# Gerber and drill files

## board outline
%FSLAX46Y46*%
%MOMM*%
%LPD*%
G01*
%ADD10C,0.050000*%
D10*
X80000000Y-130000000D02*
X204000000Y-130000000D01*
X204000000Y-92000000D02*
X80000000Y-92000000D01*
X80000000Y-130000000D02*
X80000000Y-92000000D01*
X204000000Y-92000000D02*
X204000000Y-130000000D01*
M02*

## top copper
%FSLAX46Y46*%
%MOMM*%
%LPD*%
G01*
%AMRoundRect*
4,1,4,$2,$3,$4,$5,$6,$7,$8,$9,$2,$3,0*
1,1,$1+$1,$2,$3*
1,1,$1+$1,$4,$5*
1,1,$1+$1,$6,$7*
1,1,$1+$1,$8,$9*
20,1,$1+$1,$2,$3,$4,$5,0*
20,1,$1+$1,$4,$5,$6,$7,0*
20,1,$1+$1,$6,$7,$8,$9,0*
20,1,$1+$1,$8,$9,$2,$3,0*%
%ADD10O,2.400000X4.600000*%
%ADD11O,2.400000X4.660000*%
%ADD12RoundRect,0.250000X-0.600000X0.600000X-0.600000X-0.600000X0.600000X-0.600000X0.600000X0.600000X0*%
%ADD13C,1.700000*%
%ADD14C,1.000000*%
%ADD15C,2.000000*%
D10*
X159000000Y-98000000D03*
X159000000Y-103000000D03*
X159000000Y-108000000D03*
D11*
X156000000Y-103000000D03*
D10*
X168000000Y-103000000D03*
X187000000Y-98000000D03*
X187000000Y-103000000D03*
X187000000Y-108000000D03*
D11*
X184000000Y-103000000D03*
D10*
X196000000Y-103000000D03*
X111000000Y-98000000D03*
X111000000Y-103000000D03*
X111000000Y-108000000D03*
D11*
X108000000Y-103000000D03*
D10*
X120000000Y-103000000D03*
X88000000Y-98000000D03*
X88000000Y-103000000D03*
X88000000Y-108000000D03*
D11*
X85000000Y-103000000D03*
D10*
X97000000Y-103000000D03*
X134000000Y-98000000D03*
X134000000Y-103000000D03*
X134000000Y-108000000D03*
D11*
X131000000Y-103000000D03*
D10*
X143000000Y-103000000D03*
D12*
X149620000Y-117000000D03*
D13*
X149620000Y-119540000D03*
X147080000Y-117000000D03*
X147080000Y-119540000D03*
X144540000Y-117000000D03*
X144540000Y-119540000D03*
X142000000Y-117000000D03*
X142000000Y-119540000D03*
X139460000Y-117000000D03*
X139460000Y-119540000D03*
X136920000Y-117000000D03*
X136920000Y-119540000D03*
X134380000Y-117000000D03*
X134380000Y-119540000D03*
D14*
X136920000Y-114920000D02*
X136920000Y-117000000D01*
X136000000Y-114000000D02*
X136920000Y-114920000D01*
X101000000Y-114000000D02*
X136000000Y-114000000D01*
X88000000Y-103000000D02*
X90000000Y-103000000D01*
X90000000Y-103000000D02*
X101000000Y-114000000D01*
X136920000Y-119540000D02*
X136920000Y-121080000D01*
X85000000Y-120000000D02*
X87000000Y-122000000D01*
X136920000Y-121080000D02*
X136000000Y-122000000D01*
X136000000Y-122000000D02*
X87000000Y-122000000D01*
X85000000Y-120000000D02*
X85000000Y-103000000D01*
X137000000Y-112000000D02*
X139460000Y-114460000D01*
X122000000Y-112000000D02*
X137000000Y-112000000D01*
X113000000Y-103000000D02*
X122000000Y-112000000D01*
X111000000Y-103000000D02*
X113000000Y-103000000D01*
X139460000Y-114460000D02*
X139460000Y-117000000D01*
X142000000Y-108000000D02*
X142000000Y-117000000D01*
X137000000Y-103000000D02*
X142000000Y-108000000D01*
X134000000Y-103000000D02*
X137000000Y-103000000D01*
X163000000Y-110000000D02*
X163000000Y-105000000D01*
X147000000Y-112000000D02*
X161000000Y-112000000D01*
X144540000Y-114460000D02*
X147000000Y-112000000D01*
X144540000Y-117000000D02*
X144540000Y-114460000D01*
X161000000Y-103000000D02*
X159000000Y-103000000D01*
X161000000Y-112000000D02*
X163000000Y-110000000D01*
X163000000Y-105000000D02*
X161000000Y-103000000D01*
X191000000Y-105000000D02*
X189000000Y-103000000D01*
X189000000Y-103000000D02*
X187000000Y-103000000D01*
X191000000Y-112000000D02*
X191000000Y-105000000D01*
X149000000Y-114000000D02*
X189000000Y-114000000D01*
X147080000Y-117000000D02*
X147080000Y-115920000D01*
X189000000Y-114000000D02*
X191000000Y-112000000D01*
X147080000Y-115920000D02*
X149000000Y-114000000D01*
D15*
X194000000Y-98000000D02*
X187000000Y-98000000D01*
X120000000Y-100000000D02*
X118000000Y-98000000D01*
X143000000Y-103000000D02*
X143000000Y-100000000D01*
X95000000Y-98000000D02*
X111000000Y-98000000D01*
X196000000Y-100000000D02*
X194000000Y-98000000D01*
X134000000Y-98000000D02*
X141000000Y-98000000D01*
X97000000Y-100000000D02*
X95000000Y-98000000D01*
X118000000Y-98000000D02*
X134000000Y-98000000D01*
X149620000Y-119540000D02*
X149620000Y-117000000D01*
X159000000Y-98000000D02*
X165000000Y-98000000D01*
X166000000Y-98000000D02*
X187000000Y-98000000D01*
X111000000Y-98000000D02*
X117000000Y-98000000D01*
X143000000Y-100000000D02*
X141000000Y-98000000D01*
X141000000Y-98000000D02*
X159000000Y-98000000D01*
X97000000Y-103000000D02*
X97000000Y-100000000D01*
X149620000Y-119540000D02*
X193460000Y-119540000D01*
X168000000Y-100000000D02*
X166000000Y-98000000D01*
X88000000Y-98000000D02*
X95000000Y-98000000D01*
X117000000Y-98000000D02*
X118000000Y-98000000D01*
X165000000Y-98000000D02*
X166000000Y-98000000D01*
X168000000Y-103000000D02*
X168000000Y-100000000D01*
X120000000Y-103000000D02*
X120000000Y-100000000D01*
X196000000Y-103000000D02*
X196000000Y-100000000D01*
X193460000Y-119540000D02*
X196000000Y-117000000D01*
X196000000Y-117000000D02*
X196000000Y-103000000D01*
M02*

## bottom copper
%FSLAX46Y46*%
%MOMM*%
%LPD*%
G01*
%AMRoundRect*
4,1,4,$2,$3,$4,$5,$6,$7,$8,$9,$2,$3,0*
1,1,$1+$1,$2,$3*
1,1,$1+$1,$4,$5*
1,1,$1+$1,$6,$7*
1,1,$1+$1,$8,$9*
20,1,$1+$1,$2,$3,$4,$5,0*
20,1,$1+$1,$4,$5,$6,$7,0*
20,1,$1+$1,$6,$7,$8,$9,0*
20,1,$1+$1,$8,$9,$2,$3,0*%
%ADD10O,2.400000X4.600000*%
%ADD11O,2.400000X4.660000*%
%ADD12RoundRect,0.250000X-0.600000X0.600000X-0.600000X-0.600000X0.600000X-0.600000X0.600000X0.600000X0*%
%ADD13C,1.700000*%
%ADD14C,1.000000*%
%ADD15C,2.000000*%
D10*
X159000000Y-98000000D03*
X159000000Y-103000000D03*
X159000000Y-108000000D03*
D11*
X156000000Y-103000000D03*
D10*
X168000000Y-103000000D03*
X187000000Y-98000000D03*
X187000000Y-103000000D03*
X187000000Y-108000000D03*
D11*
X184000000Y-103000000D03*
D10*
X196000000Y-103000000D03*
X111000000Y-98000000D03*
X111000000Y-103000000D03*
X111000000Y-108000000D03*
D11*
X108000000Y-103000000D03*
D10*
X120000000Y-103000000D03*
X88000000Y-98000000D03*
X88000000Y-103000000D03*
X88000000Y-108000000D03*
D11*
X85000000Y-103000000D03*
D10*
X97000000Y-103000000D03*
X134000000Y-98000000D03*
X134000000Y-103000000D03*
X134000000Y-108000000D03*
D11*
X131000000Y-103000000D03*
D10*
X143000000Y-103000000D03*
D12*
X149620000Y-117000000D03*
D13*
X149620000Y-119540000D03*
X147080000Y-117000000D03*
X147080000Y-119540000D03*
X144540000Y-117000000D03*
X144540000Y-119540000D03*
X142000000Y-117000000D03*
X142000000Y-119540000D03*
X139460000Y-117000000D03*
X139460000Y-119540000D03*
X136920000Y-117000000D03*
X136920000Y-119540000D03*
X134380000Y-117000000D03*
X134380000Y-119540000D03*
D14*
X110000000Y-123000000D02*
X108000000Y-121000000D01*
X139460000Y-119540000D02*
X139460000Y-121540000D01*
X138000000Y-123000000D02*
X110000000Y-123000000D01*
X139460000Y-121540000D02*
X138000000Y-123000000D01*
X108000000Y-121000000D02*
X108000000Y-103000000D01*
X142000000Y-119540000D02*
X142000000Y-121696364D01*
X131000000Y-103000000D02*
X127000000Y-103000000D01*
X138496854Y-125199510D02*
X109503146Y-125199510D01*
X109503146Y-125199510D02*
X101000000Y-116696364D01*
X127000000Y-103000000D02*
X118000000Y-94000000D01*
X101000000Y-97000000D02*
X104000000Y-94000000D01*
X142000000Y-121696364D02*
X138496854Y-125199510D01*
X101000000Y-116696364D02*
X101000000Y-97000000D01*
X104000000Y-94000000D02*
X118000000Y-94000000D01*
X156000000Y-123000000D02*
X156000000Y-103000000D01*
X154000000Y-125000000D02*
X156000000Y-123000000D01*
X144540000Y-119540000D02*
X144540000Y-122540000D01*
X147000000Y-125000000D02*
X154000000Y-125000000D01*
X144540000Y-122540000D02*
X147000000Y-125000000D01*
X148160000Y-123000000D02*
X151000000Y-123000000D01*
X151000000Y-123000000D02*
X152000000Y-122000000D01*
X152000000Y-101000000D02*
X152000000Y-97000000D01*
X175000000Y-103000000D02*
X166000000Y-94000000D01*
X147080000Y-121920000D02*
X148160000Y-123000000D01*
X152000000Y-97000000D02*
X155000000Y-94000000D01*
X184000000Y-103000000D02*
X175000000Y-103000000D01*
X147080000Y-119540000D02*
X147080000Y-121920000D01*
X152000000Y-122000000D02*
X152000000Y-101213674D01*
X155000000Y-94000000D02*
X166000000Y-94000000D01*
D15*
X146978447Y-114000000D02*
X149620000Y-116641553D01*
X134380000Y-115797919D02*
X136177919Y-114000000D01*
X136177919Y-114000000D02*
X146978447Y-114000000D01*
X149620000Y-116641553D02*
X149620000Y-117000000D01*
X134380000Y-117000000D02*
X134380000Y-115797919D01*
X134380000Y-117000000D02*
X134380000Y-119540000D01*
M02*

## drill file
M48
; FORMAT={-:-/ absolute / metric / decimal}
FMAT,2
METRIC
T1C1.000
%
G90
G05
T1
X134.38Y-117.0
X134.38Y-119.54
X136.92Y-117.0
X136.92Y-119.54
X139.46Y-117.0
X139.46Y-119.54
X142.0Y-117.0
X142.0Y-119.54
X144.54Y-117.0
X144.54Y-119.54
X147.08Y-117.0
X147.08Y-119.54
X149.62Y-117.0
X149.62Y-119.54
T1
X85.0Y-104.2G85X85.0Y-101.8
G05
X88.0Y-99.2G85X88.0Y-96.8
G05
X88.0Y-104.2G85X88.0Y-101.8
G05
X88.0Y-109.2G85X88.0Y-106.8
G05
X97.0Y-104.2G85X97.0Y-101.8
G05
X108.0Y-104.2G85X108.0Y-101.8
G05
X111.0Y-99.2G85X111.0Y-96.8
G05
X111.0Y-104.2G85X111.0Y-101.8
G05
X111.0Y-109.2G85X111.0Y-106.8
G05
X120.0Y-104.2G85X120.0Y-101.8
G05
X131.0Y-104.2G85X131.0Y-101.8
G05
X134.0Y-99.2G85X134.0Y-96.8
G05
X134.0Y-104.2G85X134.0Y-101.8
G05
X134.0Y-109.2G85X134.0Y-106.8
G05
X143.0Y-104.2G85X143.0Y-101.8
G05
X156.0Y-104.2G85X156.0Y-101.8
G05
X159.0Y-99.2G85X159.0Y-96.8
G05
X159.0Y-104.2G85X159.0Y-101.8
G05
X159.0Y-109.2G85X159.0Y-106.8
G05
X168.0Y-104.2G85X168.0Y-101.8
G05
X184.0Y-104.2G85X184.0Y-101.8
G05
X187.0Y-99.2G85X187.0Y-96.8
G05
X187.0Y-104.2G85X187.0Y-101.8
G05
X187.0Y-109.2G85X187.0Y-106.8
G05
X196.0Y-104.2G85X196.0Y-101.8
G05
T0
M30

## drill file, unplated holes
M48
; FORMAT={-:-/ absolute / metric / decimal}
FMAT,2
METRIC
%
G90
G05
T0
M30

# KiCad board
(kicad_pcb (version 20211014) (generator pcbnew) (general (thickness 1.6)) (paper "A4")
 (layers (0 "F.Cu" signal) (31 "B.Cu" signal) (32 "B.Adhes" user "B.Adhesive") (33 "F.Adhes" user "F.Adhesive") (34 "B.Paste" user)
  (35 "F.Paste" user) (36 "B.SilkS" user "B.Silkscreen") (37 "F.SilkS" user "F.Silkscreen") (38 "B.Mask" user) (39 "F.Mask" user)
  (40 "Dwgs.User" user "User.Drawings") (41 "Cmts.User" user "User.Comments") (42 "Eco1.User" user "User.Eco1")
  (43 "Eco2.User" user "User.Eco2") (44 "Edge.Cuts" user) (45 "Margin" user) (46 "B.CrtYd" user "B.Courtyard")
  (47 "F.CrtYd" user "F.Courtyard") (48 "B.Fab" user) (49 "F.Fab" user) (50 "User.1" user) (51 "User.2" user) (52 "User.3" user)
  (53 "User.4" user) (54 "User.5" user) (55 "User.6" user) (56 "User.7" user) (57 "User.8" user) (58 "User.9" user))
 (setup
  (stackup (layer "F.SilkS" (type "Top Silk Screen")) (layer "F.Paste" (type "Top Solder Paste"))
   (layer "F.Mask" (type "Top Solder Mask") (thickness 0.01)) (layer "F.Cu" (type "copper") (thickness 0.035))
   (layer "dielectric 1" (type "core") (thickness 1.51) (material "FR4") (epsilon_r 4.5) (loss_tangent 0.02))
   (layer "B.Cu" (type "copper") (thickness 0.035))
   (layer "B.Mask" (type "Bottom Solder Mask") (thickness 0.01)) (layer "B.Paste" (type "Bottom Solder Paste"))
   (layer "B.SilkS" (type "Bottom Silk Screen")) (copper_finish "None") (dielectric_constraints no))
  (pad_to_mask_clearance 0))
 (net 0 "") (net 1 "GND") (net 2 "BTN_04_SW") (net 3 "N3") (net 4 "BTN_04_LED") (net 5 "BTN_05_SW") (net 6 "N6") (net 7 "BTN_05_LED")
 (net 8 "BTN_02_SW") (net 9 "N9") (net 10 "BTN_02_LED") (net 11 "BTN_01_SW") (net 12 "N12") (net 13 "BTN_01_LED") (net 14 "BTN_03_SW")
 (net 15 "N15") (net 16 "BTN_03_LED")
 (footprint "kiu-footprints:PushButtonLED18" (layer "F.Cu") (at 162 103)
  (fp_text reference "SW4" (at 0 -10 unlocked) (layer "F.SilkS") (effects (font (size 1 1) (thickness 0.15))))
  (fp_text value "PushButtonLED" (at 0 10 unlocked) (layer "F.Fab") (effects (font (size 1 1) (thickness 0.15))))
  (pad "1" thru_hole oval (at -3 -5 90) (size 4.6 2.4) (drill oval 3.4 1) (layers *.Cu *.Mask) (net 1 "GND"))
  (pad "2" thru_hole oval (at -3 0 90) (size 4.6 2.4) (drill oval 3.4 1) (layers *.Cu *.Mask) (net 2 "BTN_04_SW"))
  (pad "3" thru_hole oval (at -3 5 90) (size 4.6 2.4) (drill oval 3.4 1) (layers *.Cu *.Mask) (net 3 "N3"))
  (pad "4" thru_hole oval (at -6 0 90) (size 4.66 2.4) (drill oval 3.4 1) (layers *.Cu *.Mask) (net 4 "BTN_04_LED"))
  (pad "5" thru_hole oval (at 6 0 90) (size 4.6 2.4) (drill oval 3.4 1) (layers *.Cu *.Mask) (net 1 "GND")))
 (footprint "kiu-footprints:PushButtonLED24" (layer "F.Cu") (at 190 103)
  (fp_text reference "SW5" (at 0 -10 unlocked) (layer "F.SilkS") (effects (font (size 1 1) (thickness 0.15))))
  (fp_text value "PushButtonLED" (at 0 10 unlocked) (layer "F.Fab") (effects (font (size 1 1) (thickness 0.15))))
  (pad "1" thru_hole oval (at -3 -5 90) (size 4.6 2.4) (drill oval 3.4 1) (layers *.Cu *.Mask) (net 1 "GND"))
  (pad "2" thru_hole oval (at -3 0 90) (size 4.6 2.4) (drill oval 3.4 1) (layers *.Cu *.Mask) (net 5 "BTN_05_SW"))
  (pad "3" thru_hole oval (at -3 5 90) (size 4.6 2.4) (drill oval 3.4 1) (layers *.Cu *.Mask) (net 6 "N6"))
  (pad "4" thru_hole oval (at -6 0 90) (size 4.66 2.4) (drill oval 3.4 1) (layers *.Cu *.Mask) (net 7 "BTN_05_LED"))
  (pad "5" thru_hole oval (at 6 0 90) (size 4.6 2.4) (drill oval 3.4 1) (layers *.Cu *.Mask) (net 1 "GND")))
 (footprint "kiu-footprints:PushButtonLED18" (layer "F.Cu") (at 114 103)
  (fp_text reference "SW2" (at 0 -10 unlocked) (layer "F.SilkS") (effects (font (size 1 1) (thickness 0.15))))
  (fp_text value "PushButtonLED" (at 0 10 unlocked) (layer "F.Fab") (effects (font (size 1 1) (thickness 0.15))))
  (pad "1" thru_hole oval (at -3 -5 90) (size 4.6 2.4) (drill oval 3.4 1) (layers *.Cu *.Mask) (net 1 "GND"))
  (pad "2" thru_hole oval (at -3 0 90) (size 4.6 2.4) (drill oval 3.4 1) (layers *.Cu *.Mask) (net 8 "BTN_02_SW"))
  (pad "3" thru_hole oval (at -3 5 90) (size 4.6 2.4) (drill oval 3.4 1) (layers *.Cu *.Mask) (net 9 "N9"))
  (pad "4" thru_hole oval (at -6 0 90) (size 4.66 2.4) (drill oval 3.4 1) (layers *.Cu *.Mask) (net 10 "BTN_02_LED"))
  (pad "5" thru_hole oval (at 6 0 90) (size 4.6 2.4) (drill oval 3.4 1) (layers *.Cu *.Mask) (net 1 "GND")))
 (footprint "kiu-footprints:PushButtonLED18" (layer "F.Cu") (at 91 103)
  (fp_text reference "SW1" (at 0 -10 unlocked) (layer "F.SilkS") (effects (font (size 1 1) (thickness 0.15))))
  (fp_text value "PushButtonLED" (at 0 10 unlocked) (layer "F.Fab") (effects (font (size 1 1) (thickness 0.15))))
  (pad "1" thru_hole oval (at -3 -5 90) (size 4.6 2.4) (drill oval 3.4 1) (layers *.Cu *.Mask) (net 1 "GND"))
  (pad "2" thru_hole oval (at -3 0 90) (size 4.6 2.4) (drill oval 3.4 1) (layers *.Cu *.Mask) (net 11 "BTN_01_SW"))
  (pad "3" thru_hole oval (at -3 5 90) (size 4.6 2.4) (drill oval 3.4 1) (layers *.Cu *.Mask) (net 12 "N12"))
  (pad "4" thru_hole oval (at -6 0 90) (size 4.66 2.4) (drill oval 3.4 1) (layers *.Cu *.Mask) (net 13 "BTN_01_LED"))
  (pad "5" thru_hole oval (at 6 0 90) (size 4.6 2.4) (drill oval 3.4 1) (layers *.Cu *.Mask) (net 1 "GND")))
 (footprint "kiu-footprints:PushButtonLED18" (layer "F.Cu") (at 137 103)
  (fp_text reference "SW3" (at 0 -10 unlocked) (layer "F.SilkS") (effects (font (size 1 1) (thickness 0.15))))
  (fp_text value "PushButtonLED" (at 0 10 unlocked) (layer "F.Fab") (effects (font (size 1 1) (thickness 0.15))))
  (pad "1" thru_hole oval (at -3 -5 90) (size 4.6 2.4) (drill oval 3.4 1) (layers *.Cu *.Mask) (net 1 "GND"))
  (pad "2" thru_hole oval (at -3 0 90) (size 4.6 2.4) (drill oval 3.4 1) (layers *.Cu *.Mask) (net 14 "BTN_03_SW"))
  (pad "3" thru_hole oval (at -3 5 90) (size 4.6 2.4) (drill oval 3.4 1) (layers *.Cu *.Mask) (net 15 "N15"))
  (pad "4" thru_hole oval (at -6 0 90) (size 4.66 2.4) (drill oval 3.4 1) (layers *.Cu *.Mask) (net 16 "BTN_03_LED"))
  (pad "5" thru_hole oval (at 6 0 90) (size 4.6 2.4) (drill oval 3.4 1) (layers *.Cu *.Mask) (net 1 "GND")))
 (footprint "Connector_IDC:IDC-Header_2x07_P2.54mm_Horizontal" (layer "F.Cu") (at 149.62 117 -90)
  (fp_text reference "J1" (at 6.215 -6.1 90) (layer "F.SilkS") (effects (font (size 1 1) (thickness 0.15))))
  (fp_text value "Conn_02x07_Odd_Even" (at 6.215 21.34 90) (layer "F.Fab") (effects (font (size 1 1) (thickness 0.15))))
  (pad "1" thru_hole roundrect locked (at 0 0 270) (size 1.7 1.7) (drill 1) (layers *.Cu *.Mask) (roundrect_rratio 0.1470588235)
   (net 1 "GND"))
  (pad "2" thru_hole circle locked (at 2.54 0 270) (size 1.7 1.7) (drill 1) (layers *.Cu *.Mask) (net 1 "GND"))
  (pad "3" thru_hole circle locked (at 0 2.54 270) (size 1.7 1.7) (drill 1) (layers *.Cu *.Mask) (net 5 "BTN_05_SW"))
  (pad "4" thru_hole circle locked (at 2.54 2.54 270) (size 1.7 1.7) (drill 1) (layers *.Cu *.Mask) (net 7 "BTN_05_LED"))
  (pad "5" thru_hole circle locked (at 0 5.08 270) (size 1.7 1.7) (drill 1) (layers *.Cu *.Mask) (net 2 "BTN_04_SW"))
  (pad "6" thru_hole circle locked (at 2.54 5.08 270) (size 1.7 1.7) (drill 1) (layers *.Cu *.Mask) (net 4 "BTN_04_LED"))
  (pad "7" thru_hole circle locked (at 0 7.62 270) (size 1.7 1.7) (drill 1) (layers *.Cu *.Mask) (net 14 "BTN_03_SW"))
  (pad "8" thru_hole circle locked (at 2.54 7.62 270) (size 1.7 1.7) (drill 1) (layers *.Cu *.Mask) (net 16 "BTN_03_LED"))
  (pad "9" thru_hole circle locked (at 0 10.16 270) (size 1.7 1.7) (drill 1) (layers *.Cu *.Mask) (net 8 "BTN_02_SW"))
  (pad "10" thru_hole circle locked (at 2.54 10.16 270) (size 1.7 1.7) (drill 1) (layers *.Cu *.Mask) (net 10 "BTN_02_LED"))
  (pad "11" thru_hole circle locked (at 0 12.7 270) (size 1.7 1.7) (drill 1) (layers *.Cu *.Mask) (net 11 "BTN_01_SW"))
  (pad "12" thru_hole circle locked (at 2.54 12.7 270) (size 1.7 1.7) (drill 1) (layers *.Cu *.Mask) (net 13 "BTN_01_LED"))
  (pad "13" thru_hole circle locked (at 0 15.24 270) (size 1.7 1.7) (drill 1) (layers *.Cu *.Mask) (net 1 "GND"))
  (pad "14" thru_hole circle locked (at 2.54 15.24 270) (size 1.7 1.7) (drill 1) (layers *.Cu *.Mask) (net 1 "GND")))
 (gr_line (start 80 130) (end 204 130) (layer "Edge.Cuts") (width 0.05))
 (gr_line (start 204 92) (end 80 92) (layer "Edge.Cuts") (width 0.05))
 (gr_line (start 80 130) (end 80 92) (layer "Edge.Cuts") (width 0.05))
 (gr_line (start 204 92) (end 204 130) (layer "Edge.Cuts") (width 0.05))
 (segment (start 136.92 114.92) (end 136.92 117) (width 1) (layer "F.Cu") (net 11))
 (segment (start 136 114) (end 136.92 114.92) (width 1) (layer "F.Cu") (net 11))
 (segment (start 101 114) (end 136 114) (width 1) (layer "F.Cu") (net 11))
 (segment (start 88 103) (end 90 103) (width 1) (layer "F.Cu") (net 11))
 (segment (start 90 103) (end 101 114) (width 1) (layer "F.Cu") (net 11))
 (segment (start 136.92 119.54) (end 136.92 121.08) (width 1) (layer "F.Cu") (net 13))
 (segment (start 85 120) (end 87 122) (width 1) (layer "F.Cu") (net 13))
 (segment (start 136.92 121.08) (end 136 122) (width 1) (layer "F.Cu") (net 13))
 (segment (start 136 122) (end 87 122) (width 1) (layer "F.Cu") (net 13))
 (segment (start 85 120) (end 85 103) (width 1) (layer "F.Cu") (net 13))
 (segment (start 137 112) (end 139.46 114.46) (width 1) (layer "F.Cu") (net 8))
 (segment (start 122 112) (end 137 112) (width 1) (layer "F.Cu") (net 8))
 (segment (start 113 103) (end 122 112) (width 1) (layer "F.Cu") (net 8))
 (segment (start 111 103) (end 113 103) (width 1) (layer "F.Cu") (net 8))
 (segment (start 139.46 114.46) (end 139.46 117) (width 1) (layer "F.Cu") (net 8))
 (segment (start 110 123) (end 108 121) (width 1) (layer "B.Cu") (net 10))
 (segment (start 139.46 119.54) (end 139.46 121.54) (width 1) (layer "B.Cu") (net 10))
 (segment (start 138 123) (end 110 123) (width 1) (layer "B.Cu") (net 10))
 (segment (start 139.46 121.54) (end 138 123) (width 1) (layer "B.Cu") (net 10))
 (segment (start 108 121) (end 108 103) (width 1) (layer "B.Cu") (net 10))
 (segment (start 142 108) (end 142 117) (width 1) (layer "F.Cu") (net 14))
 (segment (start 137 103) (end 142 108) (width 1) (layer "F.Cu") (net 14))
 (segment (start 134 103) (end 137 103) (width 1) (layer "F.Cu") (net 14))
 (segment (start 142 119.54) (end 142 121.696364) (width 1) (layer "B.Cu") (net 16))
 (segment (start 131 103) (end 127 103) (width 1) (layer "B.Cu") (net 16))
 (segment (start 138.496854 125.19951) (end 109.503146 125.19951) (width 1) (layer "B.Cu") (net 16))
 (segment (start 109.503146 125.19951) (end 101 116.696364) (width 1) (layer "B.Cu") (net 16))
 (segment (start 127 103) (end 118 94) (width 1) (layer "B.Cu") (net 16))
 (segment (start 101 97) (end 104 94) (width 1) (layer "B.Cu") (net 16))
 (segment (start 142 121.696364) (end 138.496854 125.19951) (width 1) (layer "B.Cu") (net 16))
 (segment (start 101 116.696364) (end 101 97) (width 1) (layer "B.Cu") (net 16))
 (segment (start 104 94) (end 118 94) (width 1) (layer "B.Cu") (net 16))
 (segment (start 163 110) (end 163 105) (width 1) (layer "F.Cu") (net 2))
 (segment (start 147 112) (end 161 112) (width 1) (layer "F.Cu") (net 2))
 (segment (start 144.54 114.46) (end 147 112) (width 1) (layer "F.Cu") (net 2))
 (segment (start 144.54 117) (end 144.54 114.46) (width 1) (layer "F.Cu") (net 2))
 (segment (start 161 103) (end 159 103) (width 1) (layer "F.Cu") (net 2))
 (segment (start 161 112) (end 163 110) (width 1) (layer "F.Cu") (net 2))
 (segment (start 163 105) (end 161 103) (width 1) (layer "F.Cu") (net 2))
 (segment (start 156 123) (end 156 103) (width 1) (layer "B.Cu") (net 4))
 (segment (start 154 125) (end 156 123) (width 1) (layer "B.Cu") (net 4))
 (segment (start 144.54 119.54) (end 144.54 122.54) (width 1) (layer "B.Cu") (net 4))
 (segment (start 147 125) (end 154 125) (width 1) (layer "B.Cu") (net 4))
 (segment (start 144.54 122.54) (end 147 125) (width 1) (layer "B.Cu") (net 4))
 (segment (start 191 105) (end 189 103) (width 1) (layer "F.Cu") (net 5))
 (segment (start 189 103) (end 187 103) (width 1) (layer "F.Cu") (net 5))
 (segment (start 191 112) (end 191 105) (width 1) (layer "F.Cu") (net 5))
 (segment (start 149 114) (end 189 114) (width 1) (layer "F.Cu") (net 5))
 (segment (start 147.08 117) (end 147.08 115.92) (width 1) (layer "F.Cu") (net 5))
 (segment (start 189 114) (end 191 112) (width 1) (layer "F.Cu") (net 5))
 (segment (start 147.08 115.92) (end 149 114) (width 1) (layer "F.Cu") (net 5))
 (segment (start 148.16 123) (end 151 123) (width 1) (layer "B.Cu") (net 7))
 (segment (start 151 123) (end 152 122) (width 1) (layer "B.Cu") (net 7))
 (segment (start 152 101) (end 152 97) (width 1) (layer "B.Cu") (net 7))
 (segment (start 175 103) (end 166 94) (width 1) (layer "B.Cu") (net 7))
 (segment (start 147.08 121.92) (end 148.16 123) (width 1) (layer "B.Cu") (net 7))
 (segment (start 152 97) (end 155 94) (width 1) (layer "B.Cu") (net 7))
 (segment (start 184 103) (end 175 103) (width 1) (layer "B.Cu") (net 7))
 (segment (start 147.08 119.54) (end 147.08 121.92) (width 1) (layer "B.Cu") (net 7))
 (segment (start 152 122) (end 152 101.213674) (width 1) (layer "B.Cu") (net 7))
 (segment (start 155 94) (end 166 94) (width 1) (layer "B.Cu") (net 7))
 (segment (start 194 98) (end 187 98) (width 2) (layer "F.Cu") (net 1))
 (segment (start 120 100) (end 118 98) (width 2) (layer "F.Cu") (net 1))
 (segment (start 143 103) (end 143 100) (width 2) (layer "F.Cu") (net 1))
 (segment (start 95 98) (end 111 98) (width 2) (layer "F.Cu") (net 1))
 (segment (start 196 100) (end 194 98) (width 2) (layer "F.Cu") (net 1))
 (segment (start 134 98) (end 141 98) (width 2) (layer "F.Cu") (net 1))
 (segment (start 97 100) (end 95 98) (width 2) (layer "F.Cu") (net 1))
 (segment (start 118 98) (end 134 98) (width 2) (layer "F.Cu") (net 1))
 (segment (start 149.62 119.54) (end 149.62 117) (width 2) (layer "F.Cu") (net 1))
 (segment (start 159 98) (end 165 98) (width 2) (layer "F.Cu") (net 1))
 (segment (start 166 98) (end 187 98) (width 2) (layer "F.Cu") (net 1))
 (segment (start 111 98) (end 117 98) (width 2) (layer "F.Cu") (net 1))
 (segment (start 143 100) (end 141 98) (width 2) (layer "F.Cu") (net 1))
 (segment (start 141 98) (end 159 98) (width 2) (layer "F.Cu") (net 1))
 (segment (start 97 103) (end 97 100) (width 2) (layer "F.Cu") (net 1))
 (segment (start 149.62 119.54) (end 193.46 119.54) (width 2) (layer "F.Cu") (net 1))
 (segment (start 168 100) (end 166 98) (width 2) (layer "F.Cu") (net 1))
 (segment (start 88 98) (end 95 98) (width 2) (layer "F.Cu") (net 1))
 (segment (start 117 98) (end 118 98) (width 2) (layer "F.Cu") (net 1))
 (segment (start 165 98) (end 166 98) (width 2) (layer "F.Cu") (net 1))
 (segment (start 168 103) (end 168 100) (width 2) (layer "F.Cu") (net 1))
 (segment (start 120 103) (end 120 100) (width 2) (layer "F.Cu") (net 1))
 (segment (start 196 103) (end 196 100) (width 2) (layer "F.Cu") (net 1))
 (segment (start 193.46 119.54) (end 196 117) (width 2) (layer "F.Cu") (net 1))
 (segment (start 196 117) (end 196 103) (width 2) (layer "F.Cu") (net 1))
 (segment (start 146.978447 114) (end 149.62 116.641553) (width 2) (layer "B.Cu") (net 1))
 (segment (start 134.38 115.797919) (end 136.177919 114) (width 2) (layer "B.Cu") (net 1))
 (segment (start 136.177919 114) (end 146.978447 114) (width 2) (layer "B.Cu") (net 1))
 (segment (start 149.62 116.641553) (end 149.62 117) (width 2) (layer "B.Cu") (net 1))
 (segment (start 134.38 117) (end 134.38 115.797919) (width 2) (layer "B.Cu") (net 1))
 (segment (start 134.38 117) (end 134.38 119.54) (width 2) (layer "B.Cu") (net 1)))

